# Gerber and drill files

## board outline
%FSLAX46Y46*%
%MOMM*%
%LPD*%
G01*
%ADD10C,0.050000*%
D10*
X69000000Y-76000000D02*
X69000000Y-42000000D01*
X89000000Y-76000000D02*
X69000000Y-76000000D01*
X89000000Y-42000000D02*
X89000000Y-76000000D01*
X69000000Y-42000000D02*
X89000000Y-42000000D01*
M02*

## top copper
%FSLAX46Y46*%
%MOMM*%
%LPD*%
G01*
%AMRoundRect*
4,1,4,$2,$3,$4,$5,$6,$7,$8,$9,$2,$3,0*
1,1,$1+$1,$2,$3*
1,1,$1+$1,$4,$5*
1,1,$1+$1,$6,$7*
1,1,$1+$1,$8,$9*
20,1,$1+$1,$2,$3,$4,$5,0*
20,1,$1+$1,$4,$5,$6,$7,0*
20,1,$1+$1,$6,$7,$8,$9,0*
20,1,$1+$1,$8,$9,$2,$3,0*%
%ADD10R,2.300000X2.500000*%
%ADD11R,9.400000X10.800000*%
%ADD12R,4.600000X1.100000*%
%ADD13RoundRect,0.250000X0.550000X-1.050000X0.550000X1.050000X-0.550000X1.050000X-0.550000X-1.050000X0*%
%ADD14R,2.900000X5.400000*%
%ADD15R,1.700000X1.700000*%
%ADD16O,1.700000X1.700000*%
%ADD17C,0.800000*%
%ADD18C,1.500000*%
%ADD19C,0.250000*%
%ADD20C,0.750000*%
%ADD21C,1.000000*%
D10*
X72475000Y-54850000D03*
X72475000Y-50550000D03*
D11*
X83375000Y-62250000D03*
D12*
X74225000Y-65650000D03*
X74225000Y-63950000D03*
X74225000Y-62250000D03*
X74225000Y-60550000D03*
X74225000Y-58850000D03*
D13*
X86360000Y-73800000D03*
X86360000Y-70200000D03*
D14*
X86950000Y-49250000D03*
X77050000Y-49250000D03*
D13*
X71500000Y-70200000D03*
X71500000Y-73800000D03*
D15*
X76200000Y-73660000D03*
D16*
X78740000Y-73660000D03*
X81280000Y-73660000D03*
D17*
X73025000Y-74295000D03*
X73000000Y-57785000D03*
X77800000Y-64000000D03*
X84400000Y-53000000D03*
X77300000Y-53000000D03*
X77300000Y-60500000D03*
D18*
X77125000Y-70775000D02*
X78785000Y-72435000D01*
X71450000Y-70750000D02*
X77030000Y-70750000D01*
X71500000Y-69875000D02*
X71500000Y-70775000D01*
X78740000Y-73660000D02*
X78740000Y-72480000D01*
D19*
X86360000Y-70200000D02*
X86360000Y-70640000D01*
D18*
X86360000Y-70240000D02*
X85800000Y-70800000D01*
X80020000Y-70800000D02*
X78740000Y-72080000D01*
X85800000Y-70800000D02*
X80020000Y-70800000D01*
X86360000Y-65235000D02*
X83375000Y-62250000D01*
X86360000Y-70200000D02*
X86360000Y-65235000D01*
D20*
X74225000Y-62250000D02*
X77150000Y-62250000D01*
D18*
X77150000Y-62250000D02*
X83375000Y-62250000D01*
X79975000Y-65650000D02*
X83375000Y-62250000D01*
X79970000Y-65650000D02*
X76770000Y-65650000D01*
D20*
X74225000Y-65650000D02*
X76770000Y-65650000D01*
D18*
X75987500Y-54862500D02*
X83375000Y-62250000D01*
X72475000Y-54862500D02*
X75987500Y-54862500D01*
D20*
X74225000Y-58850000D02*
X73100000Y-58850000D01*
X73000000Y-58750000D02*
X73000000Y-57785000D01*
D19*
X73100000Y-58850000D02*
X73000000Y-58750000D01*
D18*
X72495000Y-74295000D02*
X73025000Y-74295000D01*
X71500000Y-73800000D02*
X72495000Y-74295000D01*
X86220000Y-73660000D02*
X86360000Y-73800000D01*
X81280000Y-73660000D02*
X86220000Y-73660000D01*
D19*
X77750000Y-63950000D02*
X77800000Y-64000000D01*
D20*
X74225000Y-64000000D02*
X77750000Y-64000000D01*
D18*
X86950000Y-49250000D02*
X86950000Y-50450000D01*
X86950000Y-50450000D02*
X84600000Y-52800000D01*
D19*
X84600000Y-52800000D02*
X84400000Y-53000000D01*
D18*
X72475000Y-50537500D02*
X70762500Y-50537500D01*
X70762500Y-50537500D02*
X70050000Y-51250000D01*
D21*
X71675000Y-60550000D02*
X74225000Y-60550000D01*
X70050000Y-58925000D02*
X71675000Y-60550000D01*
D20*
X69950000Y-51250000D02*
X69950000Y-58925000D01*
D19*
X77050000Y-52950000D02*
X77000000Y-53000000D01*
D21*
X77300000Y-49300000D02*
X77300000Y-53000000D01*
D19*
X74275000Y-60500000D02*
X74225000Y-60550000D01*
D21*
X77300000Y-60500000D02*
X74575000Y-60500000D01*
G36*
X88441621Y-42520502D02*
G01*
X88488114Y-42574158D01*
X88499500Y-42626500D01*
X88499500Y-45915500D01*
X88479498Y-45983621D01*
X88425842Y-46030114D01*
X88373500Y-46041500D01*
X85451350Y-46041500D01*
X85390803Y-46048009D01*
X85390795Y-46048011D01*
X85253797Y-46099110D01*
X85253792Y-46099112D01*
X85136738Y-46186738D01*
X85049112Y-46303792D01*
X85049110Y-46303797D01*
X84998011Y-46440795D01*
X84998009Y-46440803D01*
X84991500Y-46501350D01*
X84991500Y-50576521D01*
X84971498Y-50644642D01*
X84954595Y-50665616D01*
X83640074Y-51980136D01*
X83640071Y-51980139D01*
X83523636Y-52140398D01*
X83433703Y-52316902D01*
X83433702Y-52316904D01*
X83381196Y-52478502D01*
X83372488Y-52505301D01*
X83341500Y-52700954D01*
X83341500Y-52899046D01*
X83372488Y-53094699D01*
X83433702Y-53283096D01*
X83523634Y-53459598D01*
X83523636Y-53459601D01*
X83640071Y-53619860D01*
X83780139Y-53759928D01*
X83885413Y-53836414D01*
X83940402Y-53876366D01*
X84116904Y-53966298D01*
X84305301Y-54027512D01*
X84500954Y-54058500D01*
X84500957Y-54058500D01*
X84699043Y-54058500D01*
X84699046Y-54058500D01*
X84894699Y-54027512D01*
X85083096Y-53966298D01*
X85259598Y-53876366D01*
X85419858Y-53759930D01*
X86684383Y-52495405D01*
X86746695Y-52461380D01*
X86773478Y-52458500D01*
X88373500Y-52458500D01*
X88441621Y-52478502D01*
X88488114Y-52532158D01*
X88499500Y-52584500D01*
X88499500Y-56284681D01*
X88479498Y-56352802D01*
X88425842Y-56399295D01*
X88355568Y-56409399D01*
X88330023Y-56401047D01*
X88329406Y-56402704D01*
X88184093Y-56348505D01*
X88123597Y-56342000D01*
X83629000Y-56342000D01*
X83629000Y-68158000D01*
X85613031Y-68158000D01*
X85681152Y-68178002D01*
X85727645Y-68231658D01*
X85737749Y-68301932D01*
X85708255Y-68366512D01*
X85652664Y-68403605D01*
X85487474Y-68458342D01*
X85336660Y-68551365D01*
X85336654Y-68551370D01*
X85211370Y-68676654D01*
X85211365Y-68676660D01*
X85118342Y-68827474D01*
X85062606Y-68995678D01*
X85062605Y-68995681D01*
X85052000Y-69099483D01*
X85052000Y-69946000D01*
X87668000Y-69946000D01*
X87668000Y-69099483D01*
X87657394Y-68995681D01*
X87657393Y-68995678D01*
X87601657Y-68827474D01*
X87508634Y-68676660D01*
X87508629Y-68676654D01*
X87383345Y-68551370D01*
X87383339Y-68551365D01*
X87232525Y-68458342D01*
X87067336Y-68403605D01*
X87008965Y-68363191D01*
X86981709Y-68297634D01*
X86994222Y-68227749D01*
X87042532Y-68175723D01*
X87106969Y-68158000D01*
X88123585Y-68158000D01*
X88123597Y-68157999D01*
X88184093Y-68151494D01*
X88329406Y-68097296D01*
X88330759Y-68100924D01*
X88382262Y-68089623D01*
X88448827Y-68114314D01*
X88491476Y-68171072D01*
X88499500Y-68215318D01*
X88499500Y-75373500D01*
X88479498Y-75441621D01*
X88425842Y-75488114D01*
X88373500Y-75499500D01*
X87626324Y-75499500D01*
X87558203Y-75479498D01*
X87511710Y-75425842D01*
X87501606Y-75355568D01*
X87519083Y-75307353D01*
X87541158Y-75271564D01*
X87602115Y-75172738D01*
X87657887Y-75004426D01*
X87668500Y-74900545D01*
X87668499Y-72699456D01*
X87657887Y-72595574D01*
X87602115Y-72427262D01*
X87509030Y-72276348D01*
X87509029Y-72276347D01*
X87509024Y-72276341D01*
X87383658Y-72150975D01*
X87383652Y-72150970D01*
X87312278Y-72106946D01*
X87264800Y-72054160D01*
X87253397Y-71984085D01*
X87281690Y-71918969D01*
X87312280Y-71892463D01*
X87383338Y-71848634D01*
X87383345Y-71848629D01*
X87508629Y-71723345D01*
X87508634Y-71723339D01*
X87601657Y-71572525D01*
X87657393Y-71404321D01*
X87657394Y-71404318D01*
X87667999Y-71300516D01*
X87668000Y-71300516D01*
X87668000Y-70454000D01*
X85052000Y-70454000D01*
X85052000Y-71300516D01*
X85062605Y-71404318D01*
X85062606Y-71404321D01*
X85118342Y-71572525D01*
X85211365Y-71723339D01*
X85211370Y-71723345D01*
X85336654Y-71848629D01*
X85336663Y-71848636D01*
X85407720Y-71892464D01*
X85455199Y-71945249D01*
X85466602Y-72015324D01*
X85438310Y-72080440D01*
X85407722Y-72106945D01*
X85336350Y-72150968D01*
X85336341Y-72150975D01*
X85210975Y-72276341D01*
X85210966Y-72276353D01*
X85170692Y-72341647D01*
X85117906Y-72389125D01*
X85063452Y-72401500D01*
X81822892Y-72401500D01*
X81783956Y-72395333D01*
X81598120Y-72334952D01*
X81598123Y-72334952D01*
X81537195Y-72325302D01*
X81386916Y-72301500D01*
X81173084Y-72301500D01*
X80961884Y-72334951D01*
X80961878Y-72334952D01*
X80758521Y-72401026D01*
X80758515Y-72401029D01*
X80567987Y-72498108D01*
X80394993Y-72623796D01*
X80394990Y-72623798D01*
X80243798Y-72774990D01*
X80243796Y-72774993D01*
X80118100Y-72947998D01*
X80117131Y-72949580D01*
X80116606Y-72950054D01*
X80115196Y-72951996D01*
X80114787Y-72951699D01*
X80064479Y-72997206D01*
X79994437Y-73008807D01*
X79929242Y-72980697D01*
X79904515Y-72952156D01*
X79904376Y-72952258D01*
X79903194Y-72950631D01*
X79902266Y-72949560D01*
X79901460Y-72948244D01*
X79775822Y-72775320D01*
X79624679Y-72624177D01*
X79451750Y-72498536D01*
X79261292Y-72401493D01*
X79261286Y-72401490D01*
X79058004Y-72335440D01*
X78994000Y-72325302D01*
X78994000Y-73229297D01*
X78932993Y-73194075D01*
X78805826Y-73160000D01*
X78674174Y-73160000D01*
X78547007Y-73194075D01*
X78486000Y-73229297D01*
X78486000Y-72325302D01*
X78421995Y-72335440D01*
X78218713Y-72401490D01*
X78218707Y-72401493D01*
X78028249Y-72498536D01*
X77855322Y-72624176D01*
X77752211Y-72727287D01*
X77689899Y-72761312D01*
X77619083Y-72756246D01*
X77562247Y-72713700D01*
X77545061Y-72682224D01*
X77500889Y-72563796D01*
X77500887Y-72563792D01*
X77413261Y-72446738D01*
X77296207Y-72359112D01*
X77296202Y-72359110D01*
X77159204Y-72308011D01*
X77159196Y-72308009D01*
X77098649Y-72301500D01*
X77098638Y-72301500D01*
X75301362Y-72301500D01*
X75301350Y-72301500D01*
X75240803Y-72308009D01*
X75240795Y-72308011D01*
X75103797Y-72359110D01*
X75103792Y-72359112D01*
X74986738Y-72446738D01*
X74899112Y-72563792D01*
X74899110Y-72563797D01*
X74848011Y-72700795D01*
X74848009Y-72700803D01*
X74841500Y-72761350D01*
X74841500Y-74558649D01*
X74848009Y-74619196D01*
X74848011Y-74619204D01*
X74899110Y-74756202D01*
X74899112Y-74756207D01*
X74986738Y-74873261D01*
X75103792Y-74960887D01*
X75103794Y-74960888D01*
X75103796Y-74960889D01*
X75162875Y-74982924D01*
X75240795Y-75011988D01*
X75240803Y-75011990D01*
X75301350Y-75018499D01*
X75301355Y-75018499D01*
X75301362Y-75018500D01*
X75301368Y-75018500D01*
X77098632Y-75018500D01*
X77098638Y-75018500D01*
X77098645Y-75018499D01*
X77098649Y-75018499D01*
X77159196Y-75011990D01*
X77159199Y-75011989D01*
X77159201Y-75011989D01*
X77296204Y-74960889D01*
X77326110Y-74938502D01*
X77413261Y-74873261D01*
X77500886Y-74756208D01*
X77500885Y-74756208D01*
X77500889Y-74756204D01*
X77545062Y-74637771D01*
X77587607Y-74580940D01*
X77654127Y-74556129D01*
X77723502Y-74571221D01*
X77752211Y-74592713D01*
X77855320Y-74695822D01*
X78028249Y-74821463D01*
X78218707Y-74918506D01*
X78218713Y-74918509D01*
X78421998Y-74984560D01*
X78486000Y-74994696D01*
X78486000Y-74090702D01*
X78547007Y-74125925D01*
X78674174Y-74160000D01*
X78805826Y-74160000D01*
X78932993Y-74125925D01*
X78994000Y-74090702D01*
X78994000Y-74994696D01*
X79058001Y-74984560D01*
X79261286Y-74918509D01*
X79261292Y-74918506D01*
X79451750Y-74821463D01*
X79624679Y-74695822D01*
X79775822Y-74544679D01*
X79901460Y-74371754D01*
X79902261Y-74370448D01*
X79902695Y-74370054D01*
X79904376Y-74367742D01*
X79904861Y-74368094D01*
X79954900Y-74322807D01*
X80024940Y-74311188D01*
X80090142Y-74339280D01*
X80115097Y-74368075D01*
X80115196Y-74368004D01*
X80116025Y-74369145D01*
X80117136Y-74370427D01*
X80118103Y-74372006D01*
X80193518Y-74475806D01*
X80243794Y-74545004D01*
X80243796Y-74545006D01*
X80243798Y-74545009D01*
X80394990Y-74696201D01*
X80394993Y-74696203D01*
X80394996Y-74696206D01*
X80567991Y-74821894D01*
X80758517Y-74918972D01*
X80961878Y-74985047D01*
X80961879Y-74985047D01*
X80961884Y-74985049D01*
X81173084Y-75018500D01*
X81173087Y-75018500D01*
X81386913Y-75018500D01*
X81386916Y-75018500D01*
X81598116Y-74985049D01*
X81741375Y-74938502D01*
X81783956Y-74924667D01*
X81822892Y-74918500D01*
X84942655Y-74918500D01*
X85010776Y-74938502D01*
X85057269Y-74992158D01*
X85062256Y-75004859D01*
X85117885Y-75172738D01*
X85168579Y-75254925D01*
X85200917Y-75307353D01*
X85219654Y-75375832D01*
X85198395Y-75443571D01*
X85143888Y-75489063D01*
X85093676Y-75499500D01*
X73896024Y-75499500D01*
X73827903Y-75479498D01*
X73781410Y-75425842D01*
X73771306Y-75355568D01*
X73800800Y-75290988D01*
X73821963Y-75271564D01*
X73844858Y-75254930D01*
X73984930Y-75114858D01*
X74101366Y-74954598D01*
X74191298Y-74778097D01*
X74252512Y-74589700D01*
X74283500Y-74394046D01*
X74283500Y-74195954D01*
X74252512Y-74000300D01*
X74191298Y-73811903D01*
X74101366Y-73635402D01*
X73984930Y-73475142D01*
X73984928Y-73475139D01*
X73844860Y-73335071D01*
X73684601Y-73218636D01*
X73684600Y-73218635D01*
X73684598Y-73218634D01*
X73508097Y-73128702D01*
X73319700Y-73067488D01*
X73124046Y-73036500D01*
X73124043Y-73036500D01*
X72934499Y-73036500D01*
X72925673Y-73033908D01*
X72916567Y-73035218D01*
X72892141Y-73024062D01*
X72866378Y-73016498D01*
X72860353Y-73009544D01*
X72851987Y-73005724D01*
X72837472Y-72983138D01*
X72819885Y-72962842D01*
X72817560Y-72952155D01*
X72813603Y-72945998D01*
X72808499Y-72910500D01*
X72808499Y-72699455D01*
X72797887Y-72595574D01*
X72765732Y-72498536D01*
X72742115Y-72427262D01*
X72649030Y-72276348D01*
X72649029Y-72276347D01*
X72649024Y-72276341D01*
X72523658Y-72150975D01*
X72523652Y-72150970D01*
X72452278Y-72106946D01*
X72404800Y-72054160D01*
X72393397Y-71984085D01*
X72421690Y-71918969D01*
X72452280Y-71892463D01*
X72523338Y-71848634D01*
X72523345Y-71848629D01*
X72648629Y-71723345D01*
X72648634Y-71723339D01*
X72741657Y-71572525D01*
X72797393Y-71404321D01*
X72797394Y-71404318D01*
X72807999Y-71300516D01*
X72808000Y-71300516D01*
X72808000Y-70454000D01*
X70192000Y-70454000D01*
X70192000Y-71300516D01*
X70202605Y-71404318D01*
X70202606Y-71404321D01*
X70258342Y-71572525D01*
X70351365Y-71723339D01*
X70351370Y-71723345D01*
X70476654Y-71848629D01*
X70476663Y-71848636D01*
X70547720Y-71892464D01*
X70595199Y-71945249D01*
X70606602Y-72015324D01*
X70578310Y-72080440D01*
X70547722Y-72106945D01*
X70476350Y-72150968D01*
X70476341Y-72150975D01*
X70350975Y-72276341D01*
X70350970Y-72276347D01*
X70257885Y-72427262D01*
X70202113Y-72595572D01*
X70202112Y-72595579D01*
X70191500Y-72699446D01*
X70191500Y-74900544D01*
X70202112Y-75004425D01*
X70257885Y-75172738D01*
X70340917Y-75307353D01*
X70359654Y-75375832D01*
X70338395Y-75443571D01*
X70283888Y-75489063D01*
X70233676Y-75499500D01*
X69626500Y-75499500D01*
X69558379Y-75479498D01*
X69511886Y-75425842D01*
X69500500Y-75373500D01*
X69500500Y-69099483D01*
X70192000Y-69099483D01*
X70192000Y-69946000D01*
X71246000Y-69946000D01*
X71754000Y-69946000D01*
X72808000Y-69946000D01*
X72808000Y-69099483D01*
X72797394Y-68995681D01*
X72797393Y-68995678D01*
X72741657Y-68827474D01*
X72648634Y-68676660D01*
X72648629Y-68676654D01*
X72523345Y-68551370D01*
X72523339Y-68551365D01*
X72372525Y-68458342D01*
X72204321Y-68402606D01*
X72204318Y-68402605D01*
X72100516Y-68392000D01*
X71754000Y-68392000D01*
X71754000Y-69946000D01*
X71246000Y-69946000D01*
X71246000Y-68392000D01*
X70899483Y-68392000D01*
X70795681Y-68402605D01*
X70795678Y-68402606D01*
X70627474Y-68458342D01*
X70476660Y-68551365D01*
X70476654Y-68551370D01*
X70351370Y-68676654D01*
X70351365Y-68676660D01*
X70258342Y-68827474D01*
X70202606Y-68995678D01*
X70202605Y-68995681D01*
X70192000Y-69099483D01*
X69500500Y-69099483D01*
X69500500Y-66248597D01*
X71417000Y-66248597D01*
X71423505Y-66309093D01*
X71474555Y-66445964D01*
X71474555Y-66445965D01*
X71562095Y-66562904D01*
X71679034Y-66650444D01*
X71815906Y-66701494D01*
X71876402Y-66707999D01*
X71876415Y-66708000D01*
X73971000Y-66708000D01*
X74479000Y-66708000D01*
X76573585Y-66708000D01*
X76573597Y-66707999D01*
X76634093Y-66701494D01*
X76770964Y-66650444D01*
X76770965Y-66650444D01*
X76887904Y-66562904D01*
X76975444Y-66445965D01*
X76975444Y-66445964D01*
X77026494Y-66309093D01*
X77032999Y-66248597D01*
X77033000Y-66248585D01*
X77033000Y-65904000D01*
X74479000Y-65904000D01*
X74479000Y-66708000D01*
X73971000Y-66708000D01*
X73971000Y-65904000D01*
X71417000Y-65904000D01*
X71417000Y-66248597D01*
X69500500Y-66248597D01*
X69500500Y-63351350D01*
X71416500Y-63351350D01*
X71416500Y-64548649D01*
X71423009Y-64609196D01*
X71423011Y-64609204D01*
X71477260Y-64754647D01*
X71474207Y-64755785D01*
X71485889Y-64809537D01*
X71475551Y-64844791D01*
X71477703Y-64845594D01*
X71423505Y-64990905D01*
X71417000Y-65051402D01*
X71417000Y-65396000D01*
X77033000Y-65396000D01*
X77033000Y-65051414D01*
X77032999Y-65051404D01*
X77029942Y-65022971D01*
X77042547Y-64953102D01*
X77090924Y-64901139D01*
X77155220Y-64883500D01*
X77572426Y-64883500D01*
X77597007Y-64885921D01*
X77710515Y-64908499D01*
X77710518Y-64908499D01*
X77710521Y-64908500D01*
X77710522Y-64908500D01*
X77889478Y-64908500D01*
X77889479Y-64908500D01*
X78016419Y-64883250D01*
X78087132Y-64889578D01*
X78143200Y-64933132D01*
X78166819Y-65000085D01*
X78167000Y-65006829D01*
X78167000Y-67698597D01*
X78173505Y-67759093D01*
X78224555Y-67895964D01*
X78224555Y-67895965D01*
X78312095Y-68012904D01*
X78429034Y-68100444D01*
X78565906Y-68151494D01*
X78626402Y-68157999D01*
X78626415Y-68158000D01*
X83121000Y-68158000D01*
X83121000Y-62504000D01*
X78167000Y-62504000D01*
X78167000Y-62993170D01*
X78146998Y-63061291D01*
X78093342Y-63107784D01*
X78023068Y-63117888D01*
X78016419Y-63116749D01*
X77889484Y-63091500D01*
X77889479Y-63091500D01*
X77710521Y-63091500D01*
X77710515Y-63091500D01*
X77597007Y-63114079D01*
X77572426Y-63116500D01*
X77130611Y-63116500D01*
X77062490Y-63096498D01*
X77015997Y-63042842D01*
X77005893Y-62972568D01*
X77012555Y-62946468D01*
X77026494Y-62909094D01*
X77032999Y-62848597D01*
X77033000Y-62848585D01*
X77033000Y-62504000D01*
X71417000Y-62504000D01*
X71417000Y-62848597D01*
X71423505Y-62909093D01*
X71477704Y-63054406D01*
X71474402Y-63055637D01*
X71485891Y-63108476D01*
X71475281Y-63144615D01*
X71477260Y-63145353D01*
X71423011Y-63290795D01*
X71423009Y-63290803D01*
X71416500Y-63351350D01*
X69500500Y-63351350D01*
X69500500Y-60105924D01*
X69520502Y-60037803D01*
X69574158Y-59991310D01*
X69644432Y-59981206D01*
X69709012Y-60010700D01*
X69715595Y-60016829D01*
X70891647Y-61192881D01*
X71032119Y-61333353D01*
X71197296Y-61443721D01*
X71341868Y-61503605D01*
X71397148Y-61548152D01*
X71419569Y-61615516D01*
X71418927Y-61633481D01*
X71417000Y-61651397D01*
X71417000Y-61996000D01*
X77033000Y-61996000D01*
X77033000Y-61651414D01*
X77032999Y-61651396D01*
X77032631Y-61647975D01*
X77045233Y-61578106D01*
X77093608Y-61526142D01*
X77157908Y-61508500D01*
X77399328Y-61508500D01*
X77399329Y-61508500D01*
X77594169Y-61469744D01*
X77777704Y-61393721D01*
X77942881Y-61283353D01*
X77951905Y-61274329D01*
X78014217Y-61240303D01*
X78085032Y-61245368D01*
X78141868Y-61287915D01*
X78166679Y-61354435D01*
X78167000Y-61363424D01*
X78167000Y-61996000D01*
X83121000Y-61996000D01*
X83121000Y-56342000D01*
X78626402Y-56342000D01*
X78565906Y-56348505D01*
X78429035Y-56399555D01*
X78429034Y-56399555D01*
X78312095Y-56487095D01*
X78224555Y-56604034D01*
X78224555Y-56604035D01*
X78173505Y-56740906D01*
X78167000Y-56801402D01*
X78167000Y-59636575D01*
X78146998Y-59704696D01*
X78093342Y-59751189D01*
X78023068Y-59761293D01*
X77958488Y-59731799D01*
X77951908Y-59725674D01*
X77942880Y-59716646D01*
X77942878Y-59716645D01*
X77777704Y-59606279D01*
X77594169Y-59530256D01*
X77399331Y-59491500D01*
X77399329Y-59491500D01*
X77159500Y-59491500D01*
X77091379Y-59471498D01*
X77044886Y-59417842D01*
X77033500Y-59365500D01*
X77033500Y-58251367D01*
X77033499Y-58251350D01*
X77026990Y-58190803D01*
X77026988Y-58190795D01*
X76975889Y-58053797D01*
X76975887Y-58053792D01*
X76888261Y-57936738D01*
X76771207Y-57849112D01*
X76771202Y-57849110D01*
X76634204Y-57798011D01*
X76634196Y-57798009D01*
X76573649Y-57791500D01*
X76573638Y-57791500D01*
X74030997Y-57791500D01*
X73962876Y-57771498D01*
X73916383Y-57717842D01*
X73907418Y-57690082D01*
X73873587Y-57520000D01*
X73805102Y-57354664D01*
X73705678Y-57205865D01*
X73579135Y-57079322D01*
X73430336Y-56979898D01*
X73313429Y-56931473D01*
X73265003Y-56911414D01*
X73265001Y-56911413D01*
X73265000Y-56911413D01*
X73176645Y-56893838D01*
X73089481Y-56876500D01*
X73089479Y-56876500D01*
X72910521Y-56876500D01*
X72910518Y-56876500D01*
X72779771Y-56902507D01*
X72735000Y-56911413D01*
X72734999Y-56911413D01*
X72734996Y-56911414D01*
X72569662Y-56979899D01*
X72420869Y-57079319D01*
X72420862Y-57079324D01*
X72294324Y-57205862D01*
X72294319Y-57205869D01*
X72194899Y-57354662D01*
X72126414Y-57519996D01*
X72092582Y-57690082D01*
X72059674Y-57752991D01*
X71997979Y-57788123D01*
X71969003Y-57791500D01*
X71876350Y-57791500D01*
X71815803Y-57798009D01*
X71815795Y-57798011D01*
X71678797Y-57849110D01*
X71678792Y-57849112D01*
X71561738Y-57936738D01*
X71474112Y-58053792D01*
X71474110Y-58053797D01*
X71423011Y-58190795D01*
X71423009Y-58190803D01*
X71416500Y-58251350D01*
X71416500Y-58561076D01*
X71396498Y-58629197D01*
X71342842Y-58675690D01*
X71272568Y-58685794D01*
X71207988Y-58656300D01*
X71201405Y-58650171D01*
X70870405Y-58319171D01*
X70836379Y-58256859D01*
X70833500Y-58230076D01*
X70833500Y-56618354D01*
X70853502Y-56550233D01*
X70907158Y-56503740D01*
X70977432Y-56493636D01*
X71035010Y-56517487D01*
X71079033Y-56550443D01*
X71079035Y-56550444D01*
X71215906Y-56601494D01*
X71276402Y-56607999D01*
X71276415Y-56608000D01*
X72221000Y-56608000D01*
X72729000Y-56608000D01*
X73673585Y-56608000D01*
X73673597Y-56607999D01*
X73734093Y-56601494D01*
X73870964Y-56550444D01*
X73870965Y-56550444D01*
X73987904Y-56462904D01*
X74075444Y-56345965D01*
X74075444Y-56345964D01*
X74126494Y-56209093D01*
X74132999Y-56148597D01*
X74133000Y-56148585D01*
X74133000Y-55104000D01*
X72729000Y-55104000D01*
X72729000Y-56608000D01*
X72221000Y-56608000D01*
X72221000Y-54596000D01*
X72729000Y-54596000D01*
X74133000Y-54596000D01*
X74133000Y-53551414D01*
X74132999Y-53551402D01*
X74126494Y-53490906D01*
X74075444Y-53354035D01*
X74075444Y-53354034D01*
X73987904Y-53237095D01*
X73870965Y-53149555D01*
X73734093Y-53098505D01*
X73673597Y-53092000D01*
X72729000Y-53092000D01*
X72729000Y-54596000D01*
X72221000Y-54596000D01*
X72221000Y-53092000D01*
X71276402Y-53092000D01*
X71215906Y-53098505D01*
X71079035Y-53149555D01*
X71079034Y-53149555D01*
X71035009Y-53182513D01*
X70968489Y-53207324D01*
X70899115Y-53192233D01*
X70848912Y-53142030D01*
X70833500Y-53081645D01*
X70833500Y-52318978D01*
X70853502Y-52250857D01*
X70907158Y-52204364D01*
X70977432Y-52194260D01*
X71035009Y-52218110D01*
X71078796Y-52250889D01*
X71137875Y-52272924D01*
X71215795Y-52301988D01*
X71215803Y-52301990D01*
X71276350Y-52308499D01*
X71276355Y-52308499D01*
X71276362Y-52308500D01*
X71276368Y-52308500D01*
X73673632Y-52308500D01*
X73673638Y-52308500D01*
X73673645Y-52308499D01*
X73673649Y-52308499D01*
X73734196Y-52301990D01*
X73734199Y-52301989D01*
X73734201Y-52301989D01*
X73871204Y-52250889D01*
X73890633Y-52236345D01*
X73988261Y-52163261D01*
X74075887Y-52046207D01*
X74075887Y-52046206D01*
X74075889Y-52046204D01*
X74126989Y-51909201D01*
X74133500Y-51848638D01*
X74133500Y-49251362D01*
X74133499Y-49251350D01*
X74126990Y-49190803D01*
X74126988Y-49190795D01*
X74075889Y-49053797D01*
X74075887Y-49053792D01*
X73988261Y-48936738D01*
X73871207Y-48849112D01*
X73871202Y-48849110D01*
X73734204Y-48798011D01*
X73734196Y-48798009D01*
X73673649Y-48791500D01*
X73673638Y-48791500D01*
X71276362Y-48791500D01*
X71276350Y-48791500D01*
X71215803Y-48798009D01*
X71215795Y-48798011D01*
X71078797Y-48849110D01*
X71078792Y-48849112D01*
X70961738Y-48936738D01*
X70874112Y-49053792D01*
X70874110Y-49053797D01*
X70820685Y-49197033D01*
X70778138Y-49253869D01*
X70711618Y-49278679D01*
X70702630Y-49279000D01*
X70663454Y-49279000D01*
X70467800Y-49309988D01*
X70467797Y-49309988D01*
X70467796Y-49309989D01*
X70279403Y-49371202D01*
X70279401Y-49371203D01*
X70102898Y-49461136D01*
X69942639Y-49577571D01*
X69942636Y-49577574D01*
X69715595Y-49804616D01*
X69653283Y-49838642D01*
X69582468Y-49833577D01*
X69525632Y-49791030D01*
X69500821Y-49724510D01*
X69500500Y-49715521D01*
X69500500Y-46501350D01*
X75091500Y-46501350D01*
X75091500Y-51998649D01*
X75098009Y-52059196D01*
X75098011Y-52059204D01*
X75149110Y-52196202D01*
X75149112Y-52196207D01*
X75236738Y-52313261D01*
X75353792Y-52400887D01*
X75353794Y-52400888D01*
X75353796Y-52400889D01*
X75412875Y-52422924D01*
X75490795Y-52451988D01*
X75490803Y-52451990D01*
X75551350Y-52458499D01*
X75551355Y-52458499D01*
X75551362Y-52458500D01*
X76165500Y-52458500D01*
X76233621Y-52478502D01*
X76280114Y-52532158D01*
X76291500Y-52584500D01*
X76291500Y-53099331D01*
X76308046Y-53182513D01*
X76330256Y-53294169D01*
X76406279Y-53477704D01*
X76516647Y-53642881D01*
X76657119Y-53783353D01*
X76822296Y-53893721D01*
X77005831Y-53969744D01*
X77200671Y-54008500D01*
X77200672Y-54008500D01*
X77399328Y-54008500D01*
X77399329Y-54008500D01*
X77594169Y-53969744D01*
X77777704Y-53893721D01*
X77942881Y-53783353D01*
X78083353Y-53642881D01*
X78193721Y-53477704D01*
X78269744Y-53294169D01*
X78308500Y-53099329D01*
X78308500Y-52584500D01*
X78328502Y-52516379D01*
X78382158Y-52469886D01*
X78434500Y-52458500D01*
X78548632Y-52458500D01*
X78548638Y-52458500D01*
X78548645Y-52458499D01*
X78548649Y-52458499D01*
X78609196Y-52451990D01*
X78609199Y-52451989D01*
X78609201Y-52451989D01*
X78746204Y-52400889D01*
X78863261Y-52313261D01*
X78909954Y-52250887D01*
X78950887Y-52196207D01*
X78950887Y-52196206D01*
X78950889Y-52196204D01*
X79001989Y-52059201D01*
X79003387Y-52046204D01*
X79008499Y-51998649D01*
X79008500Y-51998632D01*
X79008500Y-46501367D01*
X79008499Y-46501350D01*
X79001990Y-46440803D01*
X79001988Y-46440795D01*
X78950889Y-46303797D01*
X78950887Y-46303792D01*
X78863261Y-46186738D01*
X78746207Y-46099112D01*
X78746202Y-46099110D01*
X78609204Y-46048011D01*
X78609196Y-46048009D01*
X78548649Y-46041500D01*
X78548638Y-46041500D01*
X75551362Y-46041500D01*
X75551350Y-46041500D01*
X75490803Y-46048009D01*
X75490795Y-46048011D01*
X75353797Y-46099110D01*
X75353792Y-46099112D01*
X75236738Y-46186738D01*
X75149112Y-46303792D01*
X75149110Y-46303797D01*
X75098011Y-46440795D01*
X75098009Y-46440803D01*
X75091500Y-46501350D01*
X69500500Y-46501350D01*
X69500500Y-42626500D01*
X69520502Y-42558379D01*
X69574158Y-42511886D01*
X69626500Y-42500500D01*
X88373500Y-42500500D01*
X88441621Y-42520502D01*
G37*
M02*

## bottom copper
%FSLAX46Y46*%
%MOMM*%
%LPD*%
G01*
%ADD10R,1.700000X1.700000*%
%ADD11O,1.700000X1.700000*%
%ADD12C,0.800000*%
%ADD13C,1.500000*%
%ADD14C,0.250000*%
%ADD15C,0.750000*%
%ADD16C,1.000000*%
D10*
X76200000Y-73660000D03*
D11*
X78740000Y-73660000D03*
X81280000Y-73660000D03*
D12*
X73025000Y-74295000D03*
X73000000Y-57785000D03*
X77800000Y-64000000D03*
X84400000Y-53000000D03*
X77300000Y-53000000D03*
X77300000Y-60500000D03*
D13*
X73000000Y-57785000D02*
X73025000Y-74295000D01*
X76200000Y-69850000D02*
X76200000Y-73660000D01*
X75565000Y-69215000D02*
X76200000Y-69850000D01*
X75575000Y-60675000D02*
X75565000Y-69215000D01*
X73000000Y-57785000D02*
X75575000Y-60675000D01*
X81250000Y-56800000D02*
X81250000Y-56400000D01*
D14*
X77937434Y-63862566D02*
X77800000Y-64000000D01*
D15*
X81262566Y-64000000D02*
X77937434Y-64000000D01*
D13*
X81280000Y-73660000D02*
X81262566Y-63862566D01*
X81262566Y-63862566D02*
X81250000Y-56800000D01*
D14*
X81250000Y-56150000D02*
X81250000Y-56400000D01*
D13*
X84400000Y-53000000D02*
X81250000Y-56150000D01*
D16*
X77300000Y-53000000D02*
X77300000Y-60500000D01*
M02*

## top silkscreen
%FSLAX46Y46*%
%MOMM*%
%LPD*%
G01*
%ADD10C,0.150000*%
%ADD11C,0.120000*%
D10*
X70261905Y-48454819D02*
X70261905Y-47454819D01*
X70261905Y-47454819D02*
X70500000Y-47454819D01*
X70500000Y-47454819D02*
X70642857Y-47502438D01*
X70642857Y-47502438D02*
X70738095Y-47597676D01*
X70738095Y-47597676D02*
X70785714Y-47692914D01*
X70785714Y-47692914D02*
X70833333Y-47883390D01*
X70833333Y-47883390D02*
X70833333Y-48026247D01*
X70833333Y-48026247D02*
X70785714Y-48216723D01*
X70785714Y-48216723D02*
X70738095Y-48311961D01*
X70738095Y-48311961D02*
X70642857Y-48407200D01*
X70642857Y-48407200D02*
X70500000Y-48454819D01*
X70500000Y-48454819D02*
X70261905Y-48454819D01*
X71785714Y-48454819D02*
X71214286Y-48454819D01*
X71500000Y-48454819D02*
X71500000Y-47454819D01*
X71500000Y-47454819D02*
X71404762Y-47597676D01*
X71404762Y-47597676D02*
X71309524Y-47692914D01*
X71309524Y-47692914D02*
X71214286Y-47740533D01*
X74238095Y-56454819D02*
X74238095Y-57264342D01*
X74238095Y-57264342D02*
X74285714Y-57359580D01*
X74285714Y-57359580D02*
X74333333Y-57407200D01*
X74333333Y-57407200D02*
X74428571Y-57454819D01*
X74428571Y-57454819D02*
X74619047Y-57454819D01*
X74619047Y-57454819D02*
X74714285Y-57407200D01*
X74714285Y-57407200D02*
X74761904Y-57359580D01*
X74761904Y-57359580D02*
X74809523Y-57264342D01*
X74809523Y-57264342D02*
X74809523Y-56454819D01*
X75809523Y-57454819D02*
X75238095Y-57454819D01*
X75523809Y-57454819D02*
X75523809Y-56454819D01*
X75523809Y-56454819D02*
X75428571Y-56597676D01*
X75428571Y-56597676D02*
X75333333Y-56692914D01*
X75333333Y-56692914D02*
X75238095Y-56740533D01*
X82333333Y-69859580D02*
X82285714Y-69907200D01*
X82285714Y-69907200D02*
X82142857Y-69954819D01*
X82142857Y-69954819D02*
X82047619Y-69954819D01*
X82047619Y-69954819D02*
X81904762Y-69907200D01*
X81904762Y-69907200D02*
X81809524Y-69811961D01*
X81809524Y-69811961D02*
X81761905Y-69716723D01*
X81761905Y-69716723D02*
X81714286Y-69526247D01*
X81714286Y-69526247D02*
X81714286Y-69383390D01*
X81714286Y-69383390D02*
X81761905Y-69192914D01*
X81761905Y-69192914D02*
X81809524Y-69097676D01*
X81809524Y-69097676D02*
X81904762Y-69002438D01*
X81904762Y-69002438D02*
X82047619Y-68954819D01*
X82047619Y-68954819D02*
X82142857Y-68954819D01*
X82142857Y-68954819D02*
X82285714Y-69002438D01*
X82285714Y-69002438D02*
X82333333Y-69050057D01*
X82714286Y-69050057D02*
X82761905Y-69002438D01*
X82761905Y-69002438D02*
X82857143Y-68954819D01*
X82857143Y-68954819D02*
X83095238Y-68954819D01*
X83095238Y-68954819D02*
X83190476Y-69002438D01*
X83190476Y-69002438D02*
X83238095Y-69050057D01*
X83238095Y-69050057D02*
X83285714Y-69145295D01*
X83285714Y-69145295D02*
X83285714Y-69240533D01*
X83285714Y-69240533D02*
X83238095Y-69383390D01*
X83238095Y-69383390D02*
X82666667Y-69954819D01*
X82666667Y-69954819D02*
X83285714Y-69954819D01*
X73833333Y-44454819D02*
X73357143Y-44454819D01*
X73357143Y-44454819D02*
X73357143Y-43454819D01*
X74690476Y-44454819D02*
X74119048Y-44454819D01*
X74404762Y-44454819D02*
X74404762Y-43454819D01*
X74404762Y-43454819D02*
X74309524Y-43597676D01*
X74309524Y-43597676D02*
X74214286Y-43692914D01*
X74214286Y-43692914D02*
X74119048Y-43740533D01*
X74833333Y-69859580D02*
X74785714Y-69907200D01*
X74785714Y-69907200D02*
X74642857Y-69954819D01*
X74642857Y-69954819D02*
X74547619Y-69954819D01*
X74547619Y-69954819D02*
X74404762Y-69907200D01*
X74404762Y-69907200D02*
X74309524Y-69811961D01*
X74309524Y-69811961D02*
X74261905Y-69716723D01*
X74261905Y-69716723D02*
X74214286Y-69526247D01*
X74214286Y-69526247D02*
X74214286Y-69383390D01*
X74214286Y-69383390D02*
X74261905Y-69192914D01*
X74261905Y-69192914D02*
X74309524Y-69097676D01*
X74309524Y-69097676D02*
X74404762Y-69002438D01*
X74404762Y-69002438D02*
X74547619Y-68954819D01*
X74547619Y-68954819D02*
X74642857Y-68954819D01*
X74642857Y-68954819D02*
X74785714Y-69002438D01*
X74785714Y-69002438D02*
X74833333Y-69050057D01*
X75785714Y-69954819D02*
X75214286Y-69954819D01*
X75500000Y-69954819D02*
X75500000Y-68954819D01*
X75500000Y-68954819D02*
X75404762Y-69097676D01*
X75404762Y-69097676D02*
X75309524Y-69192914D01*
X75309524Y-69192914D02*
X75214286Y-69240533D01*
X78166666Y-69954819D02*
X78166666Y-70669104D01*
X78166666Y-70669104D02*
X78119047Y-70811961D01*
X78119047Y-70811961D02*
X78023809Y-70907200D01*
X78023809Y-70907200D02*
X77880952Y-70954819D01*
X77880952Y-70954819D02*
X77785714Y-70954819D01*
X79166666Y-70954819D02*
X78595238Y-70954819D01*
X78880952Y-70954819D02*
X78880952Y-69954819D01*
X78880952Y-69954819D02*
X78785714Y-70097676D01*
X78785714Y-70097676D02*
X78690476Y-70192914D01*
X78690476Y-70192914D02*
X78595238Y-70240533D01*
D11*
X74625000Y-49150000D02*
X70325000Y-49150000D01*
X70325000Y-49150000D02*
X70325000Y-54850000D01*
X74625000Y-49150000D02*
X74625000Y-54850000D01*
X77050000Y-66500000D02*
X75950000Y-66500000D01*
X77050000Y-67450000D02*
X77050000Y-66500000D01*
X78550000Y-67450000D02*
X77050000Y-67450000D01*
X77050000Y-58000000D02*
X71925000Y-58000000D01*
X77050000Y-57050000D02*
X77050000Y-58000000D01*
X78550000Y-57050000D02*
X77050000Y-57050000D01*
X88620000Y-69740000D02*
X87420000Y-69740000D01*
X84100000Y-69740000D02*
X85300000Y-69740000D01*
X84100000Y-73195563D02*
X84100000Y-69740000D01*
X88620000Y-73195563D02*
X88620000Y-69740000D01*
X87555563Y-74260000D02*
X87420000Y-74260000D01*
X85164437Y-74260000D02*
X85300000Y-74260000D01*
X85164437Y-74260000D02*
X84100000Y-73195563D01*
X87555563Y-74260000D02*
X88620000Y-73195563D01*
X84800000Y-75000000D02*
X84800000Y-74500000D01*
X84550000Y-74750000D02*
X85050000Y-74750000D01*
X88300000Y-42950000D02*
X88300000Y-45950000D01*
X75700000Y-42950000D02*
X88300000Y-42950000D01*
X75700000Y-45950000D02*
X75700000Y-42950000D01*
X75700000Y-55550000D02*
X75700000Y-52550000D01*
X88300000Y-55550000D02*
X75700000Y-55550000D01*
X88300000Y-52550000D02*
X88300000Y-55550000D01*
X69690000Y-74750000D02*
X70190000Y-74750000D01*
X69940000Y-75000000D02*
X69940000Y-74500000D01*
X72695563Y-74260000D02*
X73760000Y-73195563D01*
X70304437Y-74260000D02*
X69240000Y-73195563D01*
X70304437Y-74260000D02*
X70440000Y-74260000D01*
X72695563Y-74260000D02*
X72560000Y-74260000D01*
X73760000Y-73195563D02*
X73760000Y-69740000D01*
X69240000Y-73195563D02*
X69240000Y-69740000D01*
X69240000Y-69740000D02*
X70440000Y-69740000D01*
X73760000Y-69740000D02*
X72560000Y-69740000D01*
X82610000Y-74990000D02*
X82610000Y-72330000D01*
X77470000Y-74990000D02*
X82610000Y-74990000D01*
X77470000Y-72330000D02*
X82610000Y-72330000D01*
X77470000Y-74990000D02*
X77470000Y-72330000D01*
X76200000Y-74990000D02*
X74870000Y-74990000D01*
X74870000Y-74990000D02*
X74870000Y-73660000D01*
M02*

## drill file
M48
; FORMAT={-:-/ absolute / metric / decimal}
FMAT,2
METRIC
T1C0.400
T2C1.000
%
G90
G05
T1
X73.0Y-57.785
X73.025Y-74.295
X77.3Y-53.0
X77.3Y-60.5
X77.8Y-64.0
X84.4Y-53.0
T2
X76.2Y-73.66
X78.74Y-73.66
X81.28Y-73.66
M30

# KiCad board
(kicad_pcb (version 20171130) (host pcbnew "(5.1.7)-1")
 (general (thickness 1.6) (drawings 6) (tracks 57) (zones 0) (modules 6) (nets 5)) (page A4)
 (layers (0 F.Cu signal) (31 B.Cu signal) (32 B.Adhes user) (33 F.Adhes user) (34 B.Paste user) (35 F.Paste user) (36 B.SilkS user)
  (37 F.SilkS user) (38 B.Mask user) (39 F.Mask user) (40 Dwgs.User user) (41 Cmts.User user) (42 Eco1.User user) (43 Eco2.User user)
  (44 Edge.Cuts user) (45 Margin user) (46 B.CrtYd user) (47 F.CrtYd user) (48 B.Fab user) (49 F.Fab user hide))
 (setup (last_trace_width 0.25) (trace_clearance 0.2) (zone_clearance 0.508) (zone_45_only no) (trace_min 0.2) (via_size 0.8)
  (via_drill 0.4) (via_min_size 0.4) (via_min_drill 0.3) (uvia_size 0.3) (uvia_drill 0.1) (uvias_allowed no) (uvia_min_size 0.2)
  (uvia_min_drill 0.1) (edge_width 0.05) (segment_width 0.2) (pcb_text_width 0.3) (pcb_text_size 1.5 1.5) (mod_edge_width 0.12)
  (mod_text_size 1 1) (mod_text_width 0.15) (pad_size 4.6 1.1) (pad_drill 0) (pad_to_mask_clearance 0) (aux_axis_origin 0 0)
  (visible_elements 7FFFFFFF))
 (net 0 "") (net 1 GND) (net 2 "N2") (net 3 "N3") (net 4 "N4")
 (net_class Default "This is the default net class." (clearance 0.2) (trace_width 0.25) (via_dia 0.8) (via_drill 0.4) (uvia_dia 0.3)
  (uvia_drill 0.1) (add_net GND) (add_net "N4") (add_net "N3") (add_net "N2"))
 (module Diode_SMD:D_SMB (layer F.Cu) (at 72.475 52.7 270)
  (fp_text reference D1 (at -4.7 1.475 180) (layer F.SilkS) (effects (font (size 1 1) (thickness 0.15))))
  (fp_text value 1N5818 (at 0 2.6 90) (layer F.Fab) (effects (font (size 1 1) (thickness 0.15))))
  (fp_line (start -3.55 -2.15) (end -3.55 2.15) (layer F.SilkS) (width 0.12))
  (fp_line (start -3.55 2.15) (end 2.15 2.15) (layer F.SilkS) (width 0.12))
  (fp_line (start -3.55 -2.15) (end 2.15 -2.15) (layer F.SilkS) (width 0.12))
  (pad 2 smd rect (at 2.15 0 270) (size 2.5 2.3) (layers F.Cu F.Paste F.Mask) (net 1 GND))
  (pad 1 smd rect (at -2.15 0 270) (size 2.5 2.3) (layers F.Cu F.Paste F.Mask) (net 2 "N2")))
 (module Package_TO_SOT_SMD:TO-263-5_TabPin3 (layer F.Cu) (at 80 62.25)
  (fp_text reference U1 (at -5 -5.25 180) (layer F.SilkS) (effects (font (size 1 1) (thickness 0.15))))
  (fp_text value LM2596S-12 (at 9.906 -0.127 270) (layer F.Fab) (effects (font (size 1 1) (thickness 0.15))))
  (fp_line (start -2.95 4.25) (end -4.05 4.25) (layer F.SilkS) (width 0.12))
  (fp_line (start -2.95 5.2) (end -2.95 4.25) (layer F.SilkS) (width 0.12))
  (fp_line (start -1.45 5.2) (end -2.95 5.2) (layer F.SilkS) (width 0.12))
  (fp_line (start -2.95 -4.25) (end -8.075 -4.25) (layer F.SilkS) (width 0.12))
  (fp_line (start -2.95 -5.2) (end -2.95 -4.25) (layer F.SilkS) (width 0.12))
  (fp_line (start -1.45 -5.2) (end -2.95 -5.2) (layer F.SilkS) (width 0.12))
  (pad "" smd rect (at 0.95 2.775) (size 4.55 5.25) (layers F.Paste))
  (pad "" smd rect (at 5.8 -2.775) (size 4.55 5.25) (layers F.Paste))
  (pad "" smd rect (at 0.95 -2.775) (size 4.55 5.25) (layers F.Paste))
  (pad "" smd rect (at 5.8 2.775) (size 4.55 5.25) (layers F.Paste))
  (pad 3 smd rect (at 3.375 0) (size 9.4 10.8) (layers F.Cu F.Mask) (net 1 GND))
  (pad 5 smd rect (at -5.775 3.4) (size 4.6 1.1) (layers F.Cu F.Paste F.Mask) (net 1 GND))
  (pad FEDBACK smd rect (at -5.775 1.7) (size 4.6 1.1) (layers F.Cu F.Paste F.Mask) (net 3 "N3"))
  (pad 3 smd rect (at -5.775 0) (size 4.6 1.1) (layers F.Cu F.Paste F.Mask) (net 1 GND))
  (pad OUTPUT smd rect (at -5.775 -1.7) (size 4.6 1.1) (layers F.Cu F.Paste F.Mask) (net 2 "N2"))
  (pad INPUT smd rect (at -5.775 -3.4) (size 4.6 1.1) (layers F.Cu F.Paste F.Mask) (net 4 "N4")))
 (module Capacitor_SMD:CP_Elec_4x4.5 (layer F.Cu) (at 86.36 72 90)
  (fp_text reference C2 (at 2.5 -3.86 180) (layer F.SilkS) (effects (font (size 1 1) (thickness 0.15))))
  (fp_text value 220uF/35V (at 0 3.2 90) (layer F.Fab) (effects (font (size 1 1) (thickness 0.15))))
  (fp_line (start 2.26 2.26) (end 2.26 1.06) (layer F.SilkS) (width 0.12))
  (fp_line (start 2.26 -2.26) (end 2.26 -1.06) (layer F.SilkS) (width 0.12))
  (fp_line (start -1.195563 -2.26) (end 2.26 -2.26) (layer F.SilkS) (width 0.12))
  (fp_line (start -1.195563 2.26) (end 2.26 2.26) (layer F.SilkS) (width 0.12))
  (fp_line (start -2.26 1.195563) (end -2.26 1.06) (layer F.SilkS) (width 0.12))
  (fp_line (start -2.26 -1.195563) (end -2.26 -1.06) (layer F.SilkS) (width 0.12))
  (fp_line (start -2.26 -1.195563) (end -1.195563 -2.26) (layer F.SilkS) (width 0.12))
  (fp_line (start -2.26 1.195563) (end -1.195563 2.26) (layer F.SilkS) (width 0.12))
  (fp_line (start -3 -1.56) (end -2.5 -1.56) (layer F.SilkS) (width 0.12))
  (fp_line (start -2.75 -1.81) (end -2.75 -1.31) (layer F.SilkS) (width 0.12))
  (pad 1 smd roundrect (at -1.8 0 90) (size 2.6 1.6) (layers F.Cu F.Paste F.Mask) (roundrect_rratio 0.15625) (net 3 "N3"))
  (pad 2 smd roundrect (at 1.8 0 90) (size 2.6 1.6) (layers F.Cu F.Paste F.Mask) (roundrect_rratio 0.15625) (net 1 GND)))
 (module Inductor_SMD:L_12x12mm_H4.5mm (layer F.Cu) (at 82 49.25)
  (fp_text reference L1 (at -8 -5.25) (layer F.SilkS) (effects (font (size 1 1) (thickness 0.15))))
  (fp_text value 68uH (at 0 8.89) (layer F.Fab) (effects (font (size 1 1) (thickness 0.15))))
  (fp_line (start 6.3 -6.3) (end 6.3 -3.3) (layer F.SilkS) (width 0.12))
  (fp_line (start -6.3 -6.3) (end 6.3 -6.3) (layer F.SilkS) (width 0.12))
  (fp_line (start -6.3 -3.3) (end -6.3 -6.3) (layer F.SilkS) (width 0.12))
  (fp_line (start -6.3 6.3) (end -6.3 3.3) (layer F.SilkS) (width 0.12))
  (fp_line (start 6.3 6.3) (end -6.3 6.3) (layer F.SilkS) (width 0.12))
  (fp_line (start 6.3 3.3) (end 6.3 6.3) (layer F.SilkS) (width 0.12))
  (pad 2 smd rect (at 4.95 0) (size 2.9 5.4) (layers F.Cu F.Paste F.Mask) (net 3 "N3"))
  (pad 1 smd rect (at -4.95 0) (size 2.9 5.4) (layers F.Cu F.Paste F.Mask) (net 2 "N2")))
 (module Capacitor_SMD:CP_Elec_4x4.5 (layer F.Cu) (at 71.5 72 90)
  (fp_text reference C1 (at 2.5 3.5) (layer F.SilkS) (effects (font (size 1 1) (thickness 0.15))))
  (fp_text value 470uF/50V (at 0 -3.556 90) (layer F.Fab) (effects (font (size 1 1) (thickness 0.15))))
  (fp_line (start -2.75 -1.81) (end -2.75 -1.31) (layer F.SilkS) (width 0.12))
  (fp_line (start -3 -1.56) (end -2.5 -1.56) (layer F.SilkS) (width 0.12))
  (fp_line (start -2.26 1.195563) (end -1.195563 2.26) (layer F.SilkS) (width 0.12))
  (fp_line (start -2.26 -1.195563) (end -1.195563 -2.26) (layer F.SilkS) (width 0.12))
  (fp_line (start -2.26 -1.195563) (end -2.26 -1.06) (layer F.SilkS) (width 0.12))
  (fp_line (start -2.26 1.195563) (end -2.26 1.06) (layer F.SilkS) (width 0.12))
  (fp_line (start -1.195563 2.26) (end 2.26 2.26) (layer F.SilkS) (width 0.12))
  (fp_line (start -1.195563 -2.26) (end 2.26 -2.26) (layer F.SilkS) (width 0.12))
  (fp_line (start 2.26 -2.26) (end 2.26 -1.06) (layer F.SilkS) (width 0.12))
  (fp_line (start 2.26 2.26) (end 2.26 1.06) (layer F.SilkS) (width 0.12))
  (pad 2 smd roundrect (at 1.8 0 90) (size 2.6 1.6) (layers F.Cu F.Paste F.Mask) (roundrect_rratio 0.15625) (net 1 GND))
  (pad 1 smd roundrect (at -1.8 0 90) (size 2.6 1.6) (layers F.Cu F.Paste F.Mask) (roundrect_rratio 0.15625) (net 4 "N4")))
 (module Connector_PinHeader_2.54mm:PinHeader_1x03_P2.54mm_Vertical (layer F.Cu) (at 76.2 73.66 90)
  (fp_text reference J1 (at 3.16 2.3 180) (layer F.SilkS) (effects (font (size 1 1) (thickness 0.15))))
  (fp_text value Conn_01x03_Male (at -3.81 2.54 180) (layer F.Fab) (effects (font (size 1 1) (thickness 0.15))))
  (fp_line (start -1.33 6.41) (end 1.33 6.41) (layer F.SilkS) (width 0.12))
  (fp_line (start -1.33 1.27) (end -1.33 6.41) (layer F.SilkS) (width 0.12))
  (fp_line (start 1.33 1.27) (end 1.33 6.41) (layer F.SilkS) (width 0.12))
  (fp_line (start -1.33 1.27) (end 1.33 1.27) (layer F.SilkS) (width 0.12))
  (fp_line (start -1.33 0) (end -1.33 -1.33) (layer F.SilkS) (width 0.12))
  (fp_line (start -1.33 -1.33) (end 0 -1.33) (layer F.SilkS) (width 0.12))
  (pad 1 thru_hole rect (at 0 0 90) (size 1.7 1.7) (drill 1) (layers *.Cu *.Mask) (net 4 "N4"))
  (pad 2 thru_hole oval (at 0 2.54 90) (size 1.7 1.7) (drill 1) (layers *.Cu *.Mask) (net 1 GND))
  (pad 3 thru_hole oval (at 0 5.08 90) (size 1.7 1.7) (drill 1) (layers *.Cu *.Mask) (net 3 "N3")))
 (gr_line (start 69 76) (end 69 42) (layer Edge.Cuts) (width 0.05))
 (gr_line (start 89 76) (end 69 76) (layer Edge.Cuts) (width 0.05))
 (gr_line (start 89 42) (end 89 76) (layer Edge.Cuts) (width 0.05))
 (gr_line (start 69 42) (end 89 42) (layer Edge.Cuts) (width 0.05))
 (segment (start 77.125 70.775) (end 78.785 72.435) (width 1.5) (layer F.Cu) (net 1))
 (segment (start 71.45 70.75) (end 77.03 70.75) (width 1.5) (layer F.Cu) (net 1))
 (segment (start 71.5 69.875) (end 71.5 70.775) (width 1.5) (layer F.Cu) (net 1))
 (segment (start 78.74 73.66) (end 78.74 72.48) (width 1.5) (layer F.Cu) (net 1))
 (segment (start 86.36 70.2) (end 86.36 70.64) (width 0.25) (layer F.Cu) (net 1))
 (segment (start 86.36 70.24) (end 85.8 70.8) (width 1.5) (layer F.Cu) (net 1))
 (segment (start 80.02 70.8) (end 78.74 72.08) (width 1.5) (layer F.Cu) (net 1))
 (segment (start 85.8 70.8) (end 80.02 70.8) (width 1.5) (layer F.Cu) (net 1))
 (segment (start 86.36 65.235) (end 83.375 62.25) (width 1.5) (layer F.Cu) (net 1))
 (segment (start 86.36 70.2) (end 86.36 65.235) (width 1.5) (layer F.Cu) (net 1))
 (segment (start 74.225 62.25) (end 77.15 62.25) (width 0.75) (layer F.Cu) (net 1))
 (segment (start 77.15 62.25) (end 83.375 62.25) (width 1.5) (layer F.Cu) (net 1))
 (segment (start 79.975 65.65) (end 83.375 62.25) (width 1.5) (layer F.Cu) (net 1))
 (segment (start 79.97 65.65) (end 76.77 65.65) (width 1.5) (layer F.Cu) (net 1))
 (segment (start 74.225 65.65) (end 76.77 65.65) (width 0.75) (layer F.Cu) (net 1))
 (segment (start 75.9875 54.8625) (end 83.375 62.25) (width 1.5) (layer F.Cu) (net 1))
 (segment (start 72.475 54.8625) (end 75.9875 54.8625) (width 1.5) (layer F.Cu) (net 1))
 (via (at 73.025 74.295) (size 0.8) (drill 0.4) (layers F.Cu B.Cu) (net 4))
 (segment (start 73 57.785) (end 73.025 74.295) (width 1.5) (layer B.Cu) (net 4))
 (segment (start 74.225 58.85) (end 73.1 58.85) (width 0.75) (layer F.Cu) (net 4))
 (via (at 73 57.785) (size 0.8) (drill 0.4) (layers F.Cu B.Cu) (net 4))
 (segment (start 73 58.75) (end 73 57.785) (width 0.75) (layer F.Cu) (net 4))
 (segment (start 73.1 58.85) (end 73 58.75) (width 0.25) (layer F.Cu) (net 4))
 (segment (start 76.2 69.85) (end 76.2 73.66) (width 1.5) (layer B.Cu) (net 4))
 (segment (start 75.565 69.215) (end 76.2 69.85) (width 1.5) (layer B.Cu) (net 4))
 (segment (start 75.575 60.675) (end 75.565 69.215) (width 1.5) (layer B.Cu) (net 4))
 (segment (start 73 57.785) (end 75.575 60.675) (width 1.5) (layer B.Cu) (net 4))
 (segment (start 72.495 74.295) (end 73.025 74.295) (width 1.5) (layer F.Cu) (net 4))
 (segment (start 71.5 73.8) (end 72.495 74.295) (width 1.5) (layer F.Cu) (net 4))
 (segment (start 86.22 73.66) (end 86.36 73.8) (width 1.5) (layer F.Cu) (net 3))
 (segment (start 81.28 73.66) (end 86.22 73.66) (width 1.5) (layer F.Cu) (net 3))
 (segment (start 81.25 56.8) (end 81.25 56.4) (width 1.5) (layer B.Cu) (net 3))
 (via (at 77.8 64) (size 0.8) (drill 0.4) (layers F.Cu B.Cu) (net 3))
 (segment (start 77.937434 63.862566) (end 77.8 64) (width 0.25) (layer B.Cu) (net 3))
 (segment (start 81.262566 64) (end 77.937434 64) (width 0.75) (layer B.Cu) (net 3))
 (segment (start 81.28 73.66) (end 81.262566 63.862566) (width 1.5) (layer B.Cu) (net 3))
 (segment (start 81.262566 63.862566) (end 81.25 56.8) (width 1.5) (layer B.Cu) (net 3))
 (segment (start 77.75 63.95) (end 77.8 64) (width 0.25) (layer F.Cu) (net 3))
 (segment (start 74.225 64) (end 77.75 64) (width 0.75) (layer F.Cu) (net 3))
 (segment (start 86.95 49.25) (end 86.95 50.45) (width 1.5) (layer F.Cu) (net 3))
 (segment (start 86.95 50.45) (end 84.6 52.8) (width 1.5) (layer F.Cu) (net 3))
 (via (at 84.4 53) (size 0.8) (drill 0.4) (layers F.Cu B.Cu) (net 3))
 (segment (start 84.6 52.8) (end 84.4 53) (width 0.25) (layer F.Cu) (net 3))
 (segment (start 81.25 56.15) (end 81.25 56.4) (width 0.25) (layer B.Cu) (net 3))
 (segment (start 84.4 53) (end 81.25 56.15) (width 1.5) (layer B.Cu) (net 3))
 (segment (start 72.475 50.5375) (end 70.7625 50.5375) (width 1.5) (layer F.Cu) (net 2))
 (segment (start 70.7625 50.5375) (end 70.05 51.25) (width 1.5) (layer F.Cu) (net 2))
 (segment (start 71.675 60.55) (end 74.225 60.55) (width 1) (layer F.Cu) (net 2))
 (segment (start 70.05 58.925) (end 71.675 60.55) (width 1) (layer F.Cu) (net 2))
 (segment (start 69.95 51.25) (end 69.95 58.925) (width 0.75) (layer F.Cu) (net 2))
 (via (at 77.3 53) (size 0.8) (drill 0.4) (layers F.Cu B.Cu) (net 2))
 (segment (start 77.05 52.95) (end 77 53) (width 0.25) (layer F.Cu) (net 2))
 (segment (start 77.3 49.3) (end 77.3 53) (width 1) (layer F.Cu) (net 2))
 (via (at 77.3 60.5) (size 0.8) (drill 0.4) (layers F.Cu B.Cu) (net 2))
 (segment (start 77.3 53) (end 77.3 60.5) (width 1) (layer B.Cu) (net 2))
 (segment (start 74.275 60.5) (end 74.225 60.55) (width 0.25) (layer F.Cu) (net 2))
 (segment (start 77.3 60.5) (end 74.575 60.5) (width 1) (layer F.Cu) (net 2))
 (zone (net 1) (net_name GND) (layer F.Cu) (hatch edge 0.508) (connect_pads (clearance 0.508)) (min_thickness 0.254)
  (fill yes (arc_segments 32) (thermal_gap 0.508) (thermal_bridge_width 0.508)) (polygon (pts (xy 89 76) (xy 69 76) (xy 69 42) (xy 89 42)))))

